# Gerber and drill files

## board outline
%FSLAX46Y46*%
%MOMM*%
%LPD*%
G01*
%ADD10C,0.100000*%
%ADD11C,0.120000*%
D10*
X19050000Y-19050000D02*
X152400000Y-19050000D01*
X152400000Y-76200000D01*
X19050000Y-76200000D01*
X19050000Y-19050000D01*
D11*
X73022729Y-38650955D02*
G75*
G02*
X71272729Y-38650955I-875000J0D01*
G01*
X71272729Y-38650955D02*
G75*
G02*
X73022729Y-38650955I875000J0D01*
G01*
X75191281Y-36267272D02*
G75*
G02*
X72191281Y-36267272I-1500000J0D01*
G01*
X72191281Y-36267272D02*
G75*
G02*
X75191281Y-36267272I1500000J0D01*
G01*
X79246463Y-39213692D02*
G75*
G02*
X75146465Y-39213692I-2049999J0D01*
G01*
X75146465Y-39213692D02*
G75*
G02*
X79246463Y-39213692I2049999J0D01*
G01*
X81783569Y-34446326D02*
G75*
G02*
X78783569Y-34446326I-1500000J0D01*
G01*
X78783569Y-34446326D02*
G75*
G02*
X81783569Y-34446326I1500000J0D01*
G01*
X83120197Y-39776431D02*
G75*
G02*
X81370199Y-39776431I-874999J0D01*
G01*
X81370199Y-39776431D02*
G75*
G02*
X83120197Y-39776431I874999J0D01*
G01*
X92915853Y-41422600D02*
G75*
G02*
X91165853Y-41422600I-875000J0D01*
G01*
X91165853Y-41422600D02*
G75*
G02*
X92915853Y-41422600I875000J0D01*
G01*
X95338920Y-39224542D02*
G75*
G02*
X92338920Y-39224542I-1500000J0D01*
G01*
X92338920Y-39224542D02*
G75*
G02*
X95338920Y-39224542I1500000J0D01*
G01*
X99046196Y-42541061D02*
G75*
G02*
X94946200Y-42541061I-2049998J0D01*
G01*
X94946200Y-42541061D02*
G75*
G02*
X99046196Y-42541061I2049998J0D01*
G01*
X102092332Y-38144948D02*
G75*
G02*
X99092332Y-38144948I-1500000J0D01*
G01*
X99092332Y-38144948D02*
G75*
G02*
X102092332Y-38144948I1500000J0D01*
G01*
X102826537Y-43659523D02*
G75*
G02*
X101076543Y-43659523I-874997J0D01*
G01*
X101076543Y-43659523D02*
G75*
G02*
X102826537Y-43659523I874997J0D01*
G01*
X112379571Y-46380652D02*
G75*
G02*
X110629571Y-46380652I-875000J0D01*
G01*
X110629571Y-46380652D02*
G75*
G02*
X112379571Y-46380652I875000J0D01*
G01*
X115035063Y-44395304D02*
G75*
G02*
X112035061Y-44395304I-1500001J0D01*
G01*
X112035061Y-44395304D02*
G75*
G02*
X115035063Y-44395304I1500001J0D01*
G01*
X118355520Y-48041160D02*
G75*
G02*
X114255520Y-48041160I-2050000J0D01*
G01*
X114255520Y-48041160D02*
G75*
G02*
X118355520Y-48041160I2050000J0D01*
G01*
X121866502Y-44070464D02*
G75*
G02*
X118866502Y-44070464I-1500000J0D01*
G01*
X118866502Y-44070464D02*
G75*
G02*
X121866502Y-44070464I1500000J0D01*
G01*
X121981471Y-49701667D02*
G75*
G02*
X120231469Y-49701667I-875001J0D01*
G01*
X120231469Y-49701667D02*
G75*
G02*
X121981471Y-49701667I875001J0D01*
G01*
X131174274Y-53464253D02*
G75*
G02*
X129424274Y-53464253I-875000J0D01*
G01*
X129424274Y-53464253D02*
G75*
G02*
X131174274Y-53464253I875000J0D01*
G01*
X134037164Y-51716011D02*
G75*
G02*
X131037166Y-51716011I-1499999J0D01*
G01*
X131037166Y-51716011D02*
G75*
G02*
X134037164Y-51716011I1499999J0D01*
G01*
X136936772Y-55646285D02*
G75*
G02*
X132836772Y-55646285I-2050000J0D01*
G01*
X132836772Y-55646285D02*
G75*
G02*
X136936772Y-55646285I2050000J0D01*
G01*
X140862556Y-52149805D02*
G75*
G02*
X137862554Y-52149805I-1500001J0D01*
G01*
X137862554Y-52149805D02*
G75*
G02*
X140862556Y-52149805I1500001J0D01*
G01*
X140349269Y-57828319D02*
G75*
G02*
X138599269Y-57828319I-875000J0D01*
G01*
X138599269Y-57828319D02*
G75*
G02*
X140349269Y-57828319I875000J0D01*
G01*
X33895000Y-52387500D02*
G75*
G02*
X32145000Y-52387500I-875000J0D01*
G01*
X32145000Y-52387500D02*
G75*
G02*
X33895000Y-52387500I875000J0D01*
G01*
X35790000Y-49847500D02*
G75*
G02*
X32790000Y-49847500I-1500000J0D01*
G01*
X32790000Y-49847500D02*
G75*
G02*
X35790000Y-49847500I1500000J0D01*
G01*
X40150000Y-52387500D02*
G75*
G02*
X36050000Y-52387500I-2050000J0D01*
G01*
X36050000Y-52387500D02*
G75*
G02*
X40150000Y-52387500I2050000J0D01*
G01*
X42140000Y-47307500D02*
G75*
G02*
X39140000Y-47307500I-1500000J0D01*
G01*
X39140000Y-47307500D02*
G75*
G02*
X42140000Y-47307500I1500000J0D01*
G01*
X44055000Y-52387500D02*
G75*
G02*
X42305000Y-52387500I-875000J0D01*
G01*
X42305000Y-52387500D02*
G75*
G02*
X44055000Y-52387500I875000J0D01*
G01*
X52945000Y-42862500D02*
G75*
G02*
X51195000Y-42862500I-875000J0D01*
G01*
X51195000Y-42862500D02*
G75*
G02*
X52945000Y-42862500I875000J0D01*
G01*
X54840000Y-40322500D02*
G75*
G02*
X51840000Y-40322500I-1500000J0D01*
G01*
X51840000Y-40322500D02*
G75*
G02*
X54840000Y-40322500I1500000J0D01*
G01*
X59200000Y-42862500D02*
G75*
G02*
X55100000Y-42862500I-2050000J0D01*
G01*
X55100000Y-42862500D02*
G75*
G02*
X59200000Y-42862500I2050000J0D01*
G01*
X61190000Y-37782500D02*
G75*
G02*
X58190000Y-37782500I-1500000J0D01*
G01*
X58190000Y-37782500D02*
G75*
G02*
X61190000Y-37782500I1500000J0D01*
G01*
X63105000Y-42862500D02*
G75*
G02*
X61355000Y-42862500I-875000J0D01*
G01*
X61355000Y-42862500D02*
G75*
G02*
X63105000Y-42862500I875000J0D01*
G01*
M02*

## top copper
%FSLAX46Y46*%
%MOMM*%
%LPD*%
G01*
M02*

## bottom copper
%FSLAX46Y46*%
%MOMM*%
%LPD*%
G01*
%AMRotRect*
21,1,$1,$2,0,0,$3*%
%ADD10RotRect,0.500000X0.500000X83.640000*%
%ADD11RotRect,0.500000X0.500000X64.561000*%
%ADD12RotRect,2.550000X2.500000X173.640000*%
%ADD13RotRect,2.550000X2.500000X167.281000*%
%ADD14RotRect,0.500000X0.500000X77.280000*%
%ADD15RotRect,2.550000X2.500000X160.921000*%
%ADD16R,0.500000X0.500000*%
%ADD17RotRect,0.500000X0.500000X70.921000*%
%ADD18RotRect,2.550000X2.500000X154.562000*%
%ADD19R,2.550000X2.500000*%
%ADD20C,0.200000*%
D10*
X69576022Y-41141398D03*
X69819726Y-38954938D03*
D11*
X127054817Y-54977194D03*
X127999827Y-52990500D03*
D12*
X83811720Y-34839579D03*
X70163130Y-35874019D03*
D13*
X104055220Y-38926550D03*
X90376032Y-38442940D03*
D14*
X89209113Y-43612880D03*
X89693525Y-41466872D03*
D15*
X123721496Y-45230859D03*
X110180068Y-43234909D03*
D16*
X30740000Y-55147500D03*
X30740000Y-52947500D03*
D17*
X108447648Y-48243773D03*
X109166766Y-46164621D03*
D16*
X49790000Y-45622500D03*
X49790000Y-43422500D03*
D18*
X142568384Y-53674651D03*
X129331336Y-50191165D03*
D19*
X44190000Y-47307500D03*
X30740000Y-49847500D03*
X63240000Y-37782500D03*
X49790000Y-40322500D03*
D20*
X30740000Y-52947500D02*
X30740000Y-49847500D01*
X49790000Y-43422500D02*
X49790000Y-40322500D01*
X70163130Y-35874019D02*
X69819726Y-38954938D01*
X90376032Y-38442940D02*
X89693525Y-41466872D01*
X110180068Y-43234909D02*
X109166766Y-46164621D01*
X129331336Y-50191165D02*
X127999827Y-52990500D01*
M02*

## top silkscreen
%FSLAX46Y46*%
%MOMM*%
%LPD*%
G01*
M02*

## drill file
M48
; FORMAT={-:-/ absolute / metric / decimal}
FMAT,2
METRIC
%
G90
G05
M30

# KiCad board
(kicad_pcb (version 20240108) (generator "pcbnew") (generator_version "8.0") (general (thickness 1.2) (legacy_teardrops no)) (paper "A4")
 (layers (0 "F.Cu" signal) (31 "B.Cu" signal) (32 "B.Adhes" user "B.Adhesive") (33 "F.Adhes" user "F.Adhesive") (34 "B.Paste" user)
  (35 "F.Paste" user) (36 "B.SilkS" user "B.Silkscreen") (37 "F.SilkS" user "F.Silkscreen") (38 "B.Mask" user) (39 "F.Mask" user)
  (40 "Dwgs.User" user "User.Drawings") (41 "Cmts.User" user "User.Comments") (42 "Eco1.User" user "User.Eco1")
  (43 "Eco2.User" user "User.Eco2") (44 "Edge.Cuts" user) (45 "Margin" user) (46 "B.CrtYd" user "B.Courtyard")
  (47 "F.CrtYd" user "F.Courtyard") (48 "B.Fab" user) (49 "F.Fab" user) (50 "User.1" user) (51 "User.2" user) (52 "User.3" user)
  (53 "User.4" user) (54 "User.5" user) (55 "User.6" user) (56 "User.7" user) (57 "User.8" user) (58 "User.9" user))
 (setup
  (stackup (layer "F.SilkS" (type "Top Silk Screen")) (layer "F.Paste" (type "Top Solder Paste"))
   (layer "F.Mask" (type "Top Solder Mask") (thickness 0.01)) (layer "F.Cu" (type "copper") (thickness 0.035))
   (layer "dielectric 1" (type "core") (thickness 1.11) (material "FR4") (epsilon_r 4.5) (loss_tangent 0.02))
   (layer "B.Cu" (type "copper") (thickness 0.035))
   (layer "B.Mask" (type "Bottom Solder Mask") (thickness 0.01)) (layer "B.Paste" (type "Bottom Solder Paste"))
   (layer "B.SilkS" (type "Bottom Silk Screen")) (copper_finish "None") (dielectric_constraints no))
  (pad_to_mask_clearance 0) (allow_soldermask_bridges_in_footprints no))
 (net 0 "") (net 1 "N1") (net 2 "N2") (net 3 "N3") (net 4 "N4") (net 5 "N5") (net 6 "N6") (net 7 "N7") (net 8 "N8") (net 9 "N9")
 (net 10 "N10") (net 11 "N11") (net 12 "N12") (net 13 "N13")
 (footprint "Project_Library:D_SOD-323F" (layer "B.Cu") (at 69.697874 40.048168 83.64)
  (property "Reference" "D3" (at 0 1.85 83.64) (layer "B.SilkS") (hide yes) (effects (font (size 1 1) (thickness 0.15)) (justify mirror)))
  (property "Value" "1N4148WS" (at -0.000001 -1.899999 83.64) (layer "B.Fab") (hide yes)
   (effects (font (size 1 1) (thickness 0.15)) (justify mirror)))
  (pad "1" smd rect (at -1.1 0.000001 83.64) (size 0.5 0.5) (layers "B.Cu" "B.Paste" "B.Mask") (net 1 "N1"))
  (pad "2" smd rect (at 1.1 -0.000001 83.64) (size 0.5 0.5) (layers "B.Cu" "B.Paste" "B.Mask") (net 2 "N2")))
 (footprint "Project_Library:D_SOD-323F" (layer "B.Cu") (at 127.527322 53.983847 64.561)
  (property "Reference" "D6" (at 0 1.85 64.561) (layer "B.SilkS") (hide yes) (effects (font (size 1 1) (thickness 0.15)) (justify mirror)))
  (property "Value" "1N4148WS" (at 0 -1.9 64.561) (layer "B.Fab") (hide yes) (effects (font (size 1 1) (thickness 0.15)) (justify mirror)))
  (pad "1" smd rect (at -1.1 0 64.561) (size 0.5 0.5) (layers "B.Cu" "B.Paste" "B.Mask") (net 1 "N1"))
  (pad "2" smd rect (at 1.1 0 64.561) (size 0.5 0.5) (layers "B.Cu" "B.Paste" "B.Mask") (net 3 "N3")))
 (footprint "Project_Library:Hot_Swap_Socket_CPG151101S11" (layer "B.Cu") (at 76.987425 35.356799 -6.36)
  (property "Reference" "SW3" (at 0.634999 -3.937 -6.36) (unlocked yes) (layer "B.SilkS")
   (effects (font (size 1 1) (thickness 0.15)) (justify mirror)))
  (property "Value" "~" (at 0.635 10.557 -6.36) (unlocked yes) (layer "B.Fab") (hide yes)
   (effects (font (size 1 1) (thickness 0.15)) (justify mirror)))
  (fp_circle (center -4.445 3.81) (end -5.32 3.81) (stroke (width 0.12) (type solid)) (fill none) (layer "Edge.Cuts"))
  (fp_circle (center -3.175 1.27) (end -4.675 1.27) (stroke (width 0.12) (type solid)) (fill none) (layer "Edge.Cuts"))
  (fp_circle (center 0.635 3.809999) (end -1.414998 3.809999) (stroke (width 0.12) (type solid)) (fill none) (layer "Edge.Cuts"))
  (fp_circle (center 3.175 -1.27) (end 1.675 -1.27) (stroke (width 0.12) (type solid)) (fill none) (layer "Edge.Cuts"))
  (fp_circle (center 5.714999 3.810001) (end 4.84 3.81) (stroke (width 0.12) (type solid)) (fill none) (layer "Edge.Cuts"))
  (pad "1" smd rect (at 6.725 -1.269999 173.64) (size 2.55 2.5) (layers "B.Cu" "B.Paste" "B.Mask") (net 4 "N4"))
  (pad "2" smd rect (at -6.725 1.269999 173.64) (size 2.55 2.5) (layers "B.Cu" "B.Paste" "B.Mask") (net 2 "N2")))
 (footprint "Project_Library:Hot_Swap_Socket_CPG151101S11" (layer "B.Cu") (at 97.215626 38.684745 -12.719)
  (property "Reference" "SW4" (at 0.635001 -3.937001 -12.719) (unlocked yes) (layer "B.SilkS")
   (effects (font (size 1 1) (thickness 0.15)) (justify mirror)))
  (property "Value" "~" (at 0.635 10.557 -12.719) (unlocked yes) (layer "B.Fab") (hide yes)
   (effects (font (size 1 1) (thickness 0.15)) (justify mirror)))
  (fp_circle (center -4.445 3.810001) (end -5.32 3.809999) (stroke (width 0.12) (type solid)) (fill none) (layer "Edge.Cuts"))
  (fp_circle (center -3.175 1.27) (end -4.675 1.27) (stroke (width 0.12) (type solid)) (fill none) (layer "Edge.Cuts"))
  (fp_circle (center 0.635 3.81) (end -1.414998 3.809999) (stroke (width 0.12) (type solid)) (fill none) (layer "Edge.Cuts"))
  (fp_circle (center 3.175 -1.27) (end 1.675 -1.27) (stroke (width 0.12) (type solid)) (fill none) (layer "Edge.Cuts"))
  (fp_circle (center 5.714998 3.81) (end 4.84 3.81) (stroke (width 0.12) (type solid)) (fill none) (layer "Edge.Cuts"))
  (pad "1" smd rect (at 6.724999 -1.27 167.281) (size 2.55 2.5) (layers "B.Cu" "B.Paste" "B.Mask") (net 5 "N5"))
  (pad "2" smd rect (at -6.724999 1.27 167.281) (size 2.55 2.5) (layers "B.Cu" "B.Paste" "B.Mask") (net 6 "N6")))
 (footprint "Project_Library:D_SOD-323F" (layer "B.Cu") (at 89.451319 42.539876 77.28)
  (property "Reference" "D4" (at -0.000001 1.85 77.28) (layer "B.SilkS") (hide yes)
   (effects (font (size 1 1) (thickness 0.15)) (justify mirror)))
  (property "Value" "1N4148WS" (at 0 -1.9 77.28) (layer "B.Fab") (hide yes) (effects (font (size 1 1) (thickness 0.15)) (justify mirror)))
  (pad "1" smd rect (at -1.100001 0 77.28) (size 0.5 0.5) (layers "B.Cu" "B.Paste" "B.Mask") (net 1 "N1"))
  (pad "2" smd rect (at 1.100001 0 77.28) (size 0.5 0.5) (layers "B.Cu" "B.Paste" "B.Mask") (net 6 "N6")))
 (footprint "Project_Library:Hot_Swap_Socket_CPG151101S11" (layer "B.Cu") (at 116.950782 44.232884 -19.079)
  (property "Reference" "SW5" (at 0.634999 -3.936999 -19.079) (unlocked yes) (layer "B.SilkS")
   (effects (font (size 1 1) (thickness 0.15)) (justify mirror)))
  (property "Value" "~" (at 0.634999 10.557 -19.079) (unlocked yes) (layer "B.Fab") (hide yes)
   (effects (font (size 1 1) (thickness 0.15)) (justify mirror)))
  (fp_circle (center -4.445 3.81) (end -5.319999 3.81) (stroke (width 0.12) (type solid)) (fill none) (layer "Edge.Cuts"))
  (fp_circle (center -3.175 1.27) (end -4.675001 1.27) (stroke (width 0.12) (type solid)) (fill none) (layer "Edge.Cuts"))
  (fp_circle (center 0.635 3.810001) (end -1.415 3.809999) (stroke (width 0.12) (type solid)) (fill none) (layer "Edge.Cuts"))
  (fp_circle (center 3.175 -1.27) (end 1.675 -1.27) (stroke (width 0.12) (type solid)) (fill none) (layer "Edge.Cuts"))
  (fp_circle (center 5.715 3.81) (end 4.84 3.81) (stroke (width 0.12) (type solid)) (fill none) (layer "Edge.Cuts"))
  (pad "1" smd rect (at 6.725 -1.269999 160.921) (size 2.55 2.5) (layers "B.Cu" "B.Paste" "B.Mask") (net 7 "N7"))
  (pad "2" smd rect (at -6.725 1.269999 160.921) (size 2.55 2.5) (layers "B.Cu" "B.Paste" "B.Mask") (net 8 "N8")))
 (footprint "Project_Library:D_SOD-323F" (layer "B.Cu") (at 30.74 54.0475 90)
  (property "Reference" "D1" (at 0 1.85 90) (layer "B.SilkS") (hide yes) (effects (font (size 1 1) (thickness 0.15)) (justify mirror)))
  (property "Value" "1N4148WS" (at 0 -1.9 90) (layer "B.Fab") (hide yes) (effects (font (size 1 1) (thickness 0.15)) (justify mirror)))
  (pad "1" smd rect (at -1.1 0 90) (size 0.5 0.5) (layers "B.Cu" "B.Paste" "B.Mask") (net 1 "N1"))
  (pad "2" smd rect (at 1.1 0 90) (size 0.5 0.5) (layers "B.Cu" "B.Paste" "B.Mask") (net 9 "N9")))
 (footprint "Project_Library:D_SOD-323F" (layer "B.Cu") (at 108.807207 47.204197 70.921)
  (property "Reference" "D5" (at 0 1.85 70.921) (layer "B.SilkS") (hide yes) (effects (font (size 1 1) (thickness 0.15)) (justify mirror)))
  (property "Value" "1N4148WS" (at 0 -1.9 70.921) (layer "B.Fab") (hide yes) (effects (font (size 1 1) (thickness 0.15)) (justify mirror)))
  (pad "1" smd rect (at -1.1 0 70.921) (size 0.5 0.5) (layers "B.Cu" "B.Paste" "B.Mask") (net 1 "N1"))
  (pad "2" smd rect (at 1.1 0 70.921) (size 0.5 0.5) (layers "B.Cu" "B.Paste" "B.Mask") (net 8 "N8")))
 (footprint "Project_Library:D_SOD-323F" (layer "B.Cu") (at 49.79 44.5225 90)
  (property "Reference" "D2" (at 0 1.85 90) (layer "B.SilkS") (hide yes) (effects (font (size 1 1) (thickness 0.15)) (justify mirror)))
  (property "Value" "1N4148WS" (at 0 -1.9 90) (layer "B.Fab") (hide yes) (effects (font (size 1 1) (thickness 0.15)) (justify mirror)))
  (pad "1" smd rect (at -1.1 0 90) (size 0.5 0.5) (layers "B.Cu" "B.Paste" "B.Mask") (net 1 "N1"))
  (pad "2" smd rect (at 1.1 0 90) (size 0.5 0.5) (layers "B.Cu" "B.Paste" "B.Mask") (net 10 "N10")))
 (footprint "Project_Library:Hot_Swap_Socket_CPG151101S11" (layer "B.Cu") (at 135.94986 51.932908 -25.438)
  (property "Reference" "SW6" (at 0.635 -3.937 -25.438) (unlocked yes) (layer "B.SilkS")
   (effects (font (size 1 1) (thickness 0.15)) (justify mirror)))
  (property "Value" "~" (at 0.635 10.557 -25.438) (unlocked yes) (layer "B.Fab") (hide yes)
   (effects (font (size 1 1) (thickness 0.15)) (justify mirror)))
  (fp_circle (center -4.445 3.810002) (end -5.32 3.81) (stroke (width 0.12) (type solid)) (fill none) (layer "Edge.Cuts"))
  (fp_circle (center -3.175001 1.27) (end -4.675 1.27) (stroke (width 0.12) (type solid)) (fill none) (layer "Edge.Cuts"))
  (fp_circle (center 0.635 3.81) (end -1.415 3.81) (stroke (width 0.12) (type solid)) (fill none) (layer "Edge.Cuts"))
  (fp_circle (center 3.175001 -1.27) (end 1.675 -1.27) (stroke (width 0.12) (type solid)) (fill none) (layer "Edge.Cuts"))
  (fp_circle (center 5.715 3.81) (end 4.84 3.81) (stroke (width 0.12) (type solid)) (fill none) (layer "Edge.Cuts"))
  (pad "1" smd rect (at 6.725 -1.27 154.562) (size 2.55 2.5) (layers "B.Cu" "B.Paste" "B.Mask") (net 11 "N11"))
  (pad "2" smd rect (at -6.725 1.27 154.562) (size 2.55 2.5) (layers "B.Cu" "B.Paste" "B.Mask") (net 3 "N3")))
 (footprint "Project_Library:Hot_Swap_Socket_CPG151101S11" (layer "B.Cu") (at 37.465 48.5775)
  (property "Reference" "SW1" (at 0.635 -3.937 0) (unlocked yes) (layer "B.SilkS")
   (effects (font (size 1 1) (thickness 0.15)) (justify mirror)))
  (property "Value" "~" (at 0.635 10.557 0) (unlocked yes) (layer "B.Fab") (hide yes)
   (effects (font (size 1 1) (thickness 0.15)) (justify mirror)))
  (fp_circle (center -4.445 3.81) (end -5.32 3.81) (stroke (width 0.12) (type solid)) (fill none) (layer "Edge.Cuts"))
  (fp_circle (center -3.175 1.27) (end -4.675 1.27) (stroke (width 0.12) (type solid)) (fill none) (layer "Edge.Cuts"))
  (fp_circle (center 0.635 3.81) (end -1.415 3.81) (stroke (width 0.12) (type solid)) (fill none) (layer "Edge.Cuts"))
  (fp_circle (center 3.175 -1.27) (end 1.675 -1.27) (stroke (width 0.12) (type solid)) (fill none) (layer "Edge.Cuts"))
  (fp_circle (center 5.715 3.81) (end 4.84 3.81) (stroke (width 0.12) (type solid)) (fill none) (layer "Edge.Cuts"))
  (pad "1" smd rect (at 6.725 -1.27 180) (size 2.55 2.5) (layers "B.Cu" "B.Paste" "B.Mask") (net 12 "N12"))
  (pad "2" smd rect (at -6.725 1.27 180) (size 2.55 2.5) (layers "B.Cu" "B.Paste" "B.Mask") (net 9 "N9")))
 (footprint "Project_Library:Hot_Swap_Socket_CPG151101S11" (layer "B.Cu") (at 56.515 39.0525)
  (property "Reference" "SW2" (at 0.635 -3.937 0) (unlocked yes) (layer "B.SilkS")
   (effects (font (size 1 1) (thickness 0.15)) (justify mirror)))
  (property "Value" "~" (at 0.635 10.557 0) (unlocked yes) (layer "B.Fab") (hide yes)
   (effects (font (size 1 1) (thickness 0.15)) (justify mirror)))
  (fp_circle (center -4.445 3.81) (end -5.32 3.81) (stroke (width 0.12) (type solid)) (fill none) (layer "Edge.Cuts"))
  (fp_circle (center -3.175 1.27) (end -4.675 1.27) (stroke (width 0.12) (type solid)) (fill none) (layer "Edge.Cuts"))
  (fp_circle (center 0.635 3.81) (end -1.415 3.81) (stroke (width 0.12) (type solid)) (fill none) (layer "Edge.Cuts"))
  (fp_circle (center 3.175 -1.27) (end 1.675 -1.27) (stroke (width 0.12) (type solid)) (fill none) (layer "Edge.Cuts"))
  (fp_circle (center 5.715 3.81) (end 4.84 3.81) (stroke (width 0.12) (type solid)) (fill none) (layer "Edge.Cuts"))
  (pad "1" smd rect (at 6.725 -1.27 180) (size 2.55 2.5) (layers "B.Cu" "B.Paste" "B.Mask") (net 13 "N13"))
  (pad "2" smd rect (at -6.725 1.27 180) (size 2.55 2.5) (layers "B.Cu" "B.Paste" "B.Mask") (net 10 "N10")))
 (gr_rect (start 19.05 19.05) (end 152.4 76.2) (stroke (width 0.1) (type default)) (fill none) (layer "Edge.Cuts"))
 (segment (start 30.74 52.9475) (end 30.74 49.8475) (width 0.2) (layer "B.Cu") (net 9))
 (segment (start 49.79 43.4225) (end 49.79 40.3225) (width 0.2) (layer "B.Cu") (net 10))
 (segment (start 70.16313 35.874019) (end 69.819726 38.954938) (width 0.2) (layer "B.Cu") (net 2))
 (segment (start 90.376032 38.44294) (end 89.693525 41.466872) (width 0.2) (layer "B.Cu") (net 6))
 (segment (start 110.180068 43.234909) (end 109.166766 46.164621) (width 0.2) (layer "B.Cu") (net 8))
 (segment (start 129.331336 50.191165) (end 127.999827 52.9905) (width 0.2) (layer "B.Cu") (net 3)))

